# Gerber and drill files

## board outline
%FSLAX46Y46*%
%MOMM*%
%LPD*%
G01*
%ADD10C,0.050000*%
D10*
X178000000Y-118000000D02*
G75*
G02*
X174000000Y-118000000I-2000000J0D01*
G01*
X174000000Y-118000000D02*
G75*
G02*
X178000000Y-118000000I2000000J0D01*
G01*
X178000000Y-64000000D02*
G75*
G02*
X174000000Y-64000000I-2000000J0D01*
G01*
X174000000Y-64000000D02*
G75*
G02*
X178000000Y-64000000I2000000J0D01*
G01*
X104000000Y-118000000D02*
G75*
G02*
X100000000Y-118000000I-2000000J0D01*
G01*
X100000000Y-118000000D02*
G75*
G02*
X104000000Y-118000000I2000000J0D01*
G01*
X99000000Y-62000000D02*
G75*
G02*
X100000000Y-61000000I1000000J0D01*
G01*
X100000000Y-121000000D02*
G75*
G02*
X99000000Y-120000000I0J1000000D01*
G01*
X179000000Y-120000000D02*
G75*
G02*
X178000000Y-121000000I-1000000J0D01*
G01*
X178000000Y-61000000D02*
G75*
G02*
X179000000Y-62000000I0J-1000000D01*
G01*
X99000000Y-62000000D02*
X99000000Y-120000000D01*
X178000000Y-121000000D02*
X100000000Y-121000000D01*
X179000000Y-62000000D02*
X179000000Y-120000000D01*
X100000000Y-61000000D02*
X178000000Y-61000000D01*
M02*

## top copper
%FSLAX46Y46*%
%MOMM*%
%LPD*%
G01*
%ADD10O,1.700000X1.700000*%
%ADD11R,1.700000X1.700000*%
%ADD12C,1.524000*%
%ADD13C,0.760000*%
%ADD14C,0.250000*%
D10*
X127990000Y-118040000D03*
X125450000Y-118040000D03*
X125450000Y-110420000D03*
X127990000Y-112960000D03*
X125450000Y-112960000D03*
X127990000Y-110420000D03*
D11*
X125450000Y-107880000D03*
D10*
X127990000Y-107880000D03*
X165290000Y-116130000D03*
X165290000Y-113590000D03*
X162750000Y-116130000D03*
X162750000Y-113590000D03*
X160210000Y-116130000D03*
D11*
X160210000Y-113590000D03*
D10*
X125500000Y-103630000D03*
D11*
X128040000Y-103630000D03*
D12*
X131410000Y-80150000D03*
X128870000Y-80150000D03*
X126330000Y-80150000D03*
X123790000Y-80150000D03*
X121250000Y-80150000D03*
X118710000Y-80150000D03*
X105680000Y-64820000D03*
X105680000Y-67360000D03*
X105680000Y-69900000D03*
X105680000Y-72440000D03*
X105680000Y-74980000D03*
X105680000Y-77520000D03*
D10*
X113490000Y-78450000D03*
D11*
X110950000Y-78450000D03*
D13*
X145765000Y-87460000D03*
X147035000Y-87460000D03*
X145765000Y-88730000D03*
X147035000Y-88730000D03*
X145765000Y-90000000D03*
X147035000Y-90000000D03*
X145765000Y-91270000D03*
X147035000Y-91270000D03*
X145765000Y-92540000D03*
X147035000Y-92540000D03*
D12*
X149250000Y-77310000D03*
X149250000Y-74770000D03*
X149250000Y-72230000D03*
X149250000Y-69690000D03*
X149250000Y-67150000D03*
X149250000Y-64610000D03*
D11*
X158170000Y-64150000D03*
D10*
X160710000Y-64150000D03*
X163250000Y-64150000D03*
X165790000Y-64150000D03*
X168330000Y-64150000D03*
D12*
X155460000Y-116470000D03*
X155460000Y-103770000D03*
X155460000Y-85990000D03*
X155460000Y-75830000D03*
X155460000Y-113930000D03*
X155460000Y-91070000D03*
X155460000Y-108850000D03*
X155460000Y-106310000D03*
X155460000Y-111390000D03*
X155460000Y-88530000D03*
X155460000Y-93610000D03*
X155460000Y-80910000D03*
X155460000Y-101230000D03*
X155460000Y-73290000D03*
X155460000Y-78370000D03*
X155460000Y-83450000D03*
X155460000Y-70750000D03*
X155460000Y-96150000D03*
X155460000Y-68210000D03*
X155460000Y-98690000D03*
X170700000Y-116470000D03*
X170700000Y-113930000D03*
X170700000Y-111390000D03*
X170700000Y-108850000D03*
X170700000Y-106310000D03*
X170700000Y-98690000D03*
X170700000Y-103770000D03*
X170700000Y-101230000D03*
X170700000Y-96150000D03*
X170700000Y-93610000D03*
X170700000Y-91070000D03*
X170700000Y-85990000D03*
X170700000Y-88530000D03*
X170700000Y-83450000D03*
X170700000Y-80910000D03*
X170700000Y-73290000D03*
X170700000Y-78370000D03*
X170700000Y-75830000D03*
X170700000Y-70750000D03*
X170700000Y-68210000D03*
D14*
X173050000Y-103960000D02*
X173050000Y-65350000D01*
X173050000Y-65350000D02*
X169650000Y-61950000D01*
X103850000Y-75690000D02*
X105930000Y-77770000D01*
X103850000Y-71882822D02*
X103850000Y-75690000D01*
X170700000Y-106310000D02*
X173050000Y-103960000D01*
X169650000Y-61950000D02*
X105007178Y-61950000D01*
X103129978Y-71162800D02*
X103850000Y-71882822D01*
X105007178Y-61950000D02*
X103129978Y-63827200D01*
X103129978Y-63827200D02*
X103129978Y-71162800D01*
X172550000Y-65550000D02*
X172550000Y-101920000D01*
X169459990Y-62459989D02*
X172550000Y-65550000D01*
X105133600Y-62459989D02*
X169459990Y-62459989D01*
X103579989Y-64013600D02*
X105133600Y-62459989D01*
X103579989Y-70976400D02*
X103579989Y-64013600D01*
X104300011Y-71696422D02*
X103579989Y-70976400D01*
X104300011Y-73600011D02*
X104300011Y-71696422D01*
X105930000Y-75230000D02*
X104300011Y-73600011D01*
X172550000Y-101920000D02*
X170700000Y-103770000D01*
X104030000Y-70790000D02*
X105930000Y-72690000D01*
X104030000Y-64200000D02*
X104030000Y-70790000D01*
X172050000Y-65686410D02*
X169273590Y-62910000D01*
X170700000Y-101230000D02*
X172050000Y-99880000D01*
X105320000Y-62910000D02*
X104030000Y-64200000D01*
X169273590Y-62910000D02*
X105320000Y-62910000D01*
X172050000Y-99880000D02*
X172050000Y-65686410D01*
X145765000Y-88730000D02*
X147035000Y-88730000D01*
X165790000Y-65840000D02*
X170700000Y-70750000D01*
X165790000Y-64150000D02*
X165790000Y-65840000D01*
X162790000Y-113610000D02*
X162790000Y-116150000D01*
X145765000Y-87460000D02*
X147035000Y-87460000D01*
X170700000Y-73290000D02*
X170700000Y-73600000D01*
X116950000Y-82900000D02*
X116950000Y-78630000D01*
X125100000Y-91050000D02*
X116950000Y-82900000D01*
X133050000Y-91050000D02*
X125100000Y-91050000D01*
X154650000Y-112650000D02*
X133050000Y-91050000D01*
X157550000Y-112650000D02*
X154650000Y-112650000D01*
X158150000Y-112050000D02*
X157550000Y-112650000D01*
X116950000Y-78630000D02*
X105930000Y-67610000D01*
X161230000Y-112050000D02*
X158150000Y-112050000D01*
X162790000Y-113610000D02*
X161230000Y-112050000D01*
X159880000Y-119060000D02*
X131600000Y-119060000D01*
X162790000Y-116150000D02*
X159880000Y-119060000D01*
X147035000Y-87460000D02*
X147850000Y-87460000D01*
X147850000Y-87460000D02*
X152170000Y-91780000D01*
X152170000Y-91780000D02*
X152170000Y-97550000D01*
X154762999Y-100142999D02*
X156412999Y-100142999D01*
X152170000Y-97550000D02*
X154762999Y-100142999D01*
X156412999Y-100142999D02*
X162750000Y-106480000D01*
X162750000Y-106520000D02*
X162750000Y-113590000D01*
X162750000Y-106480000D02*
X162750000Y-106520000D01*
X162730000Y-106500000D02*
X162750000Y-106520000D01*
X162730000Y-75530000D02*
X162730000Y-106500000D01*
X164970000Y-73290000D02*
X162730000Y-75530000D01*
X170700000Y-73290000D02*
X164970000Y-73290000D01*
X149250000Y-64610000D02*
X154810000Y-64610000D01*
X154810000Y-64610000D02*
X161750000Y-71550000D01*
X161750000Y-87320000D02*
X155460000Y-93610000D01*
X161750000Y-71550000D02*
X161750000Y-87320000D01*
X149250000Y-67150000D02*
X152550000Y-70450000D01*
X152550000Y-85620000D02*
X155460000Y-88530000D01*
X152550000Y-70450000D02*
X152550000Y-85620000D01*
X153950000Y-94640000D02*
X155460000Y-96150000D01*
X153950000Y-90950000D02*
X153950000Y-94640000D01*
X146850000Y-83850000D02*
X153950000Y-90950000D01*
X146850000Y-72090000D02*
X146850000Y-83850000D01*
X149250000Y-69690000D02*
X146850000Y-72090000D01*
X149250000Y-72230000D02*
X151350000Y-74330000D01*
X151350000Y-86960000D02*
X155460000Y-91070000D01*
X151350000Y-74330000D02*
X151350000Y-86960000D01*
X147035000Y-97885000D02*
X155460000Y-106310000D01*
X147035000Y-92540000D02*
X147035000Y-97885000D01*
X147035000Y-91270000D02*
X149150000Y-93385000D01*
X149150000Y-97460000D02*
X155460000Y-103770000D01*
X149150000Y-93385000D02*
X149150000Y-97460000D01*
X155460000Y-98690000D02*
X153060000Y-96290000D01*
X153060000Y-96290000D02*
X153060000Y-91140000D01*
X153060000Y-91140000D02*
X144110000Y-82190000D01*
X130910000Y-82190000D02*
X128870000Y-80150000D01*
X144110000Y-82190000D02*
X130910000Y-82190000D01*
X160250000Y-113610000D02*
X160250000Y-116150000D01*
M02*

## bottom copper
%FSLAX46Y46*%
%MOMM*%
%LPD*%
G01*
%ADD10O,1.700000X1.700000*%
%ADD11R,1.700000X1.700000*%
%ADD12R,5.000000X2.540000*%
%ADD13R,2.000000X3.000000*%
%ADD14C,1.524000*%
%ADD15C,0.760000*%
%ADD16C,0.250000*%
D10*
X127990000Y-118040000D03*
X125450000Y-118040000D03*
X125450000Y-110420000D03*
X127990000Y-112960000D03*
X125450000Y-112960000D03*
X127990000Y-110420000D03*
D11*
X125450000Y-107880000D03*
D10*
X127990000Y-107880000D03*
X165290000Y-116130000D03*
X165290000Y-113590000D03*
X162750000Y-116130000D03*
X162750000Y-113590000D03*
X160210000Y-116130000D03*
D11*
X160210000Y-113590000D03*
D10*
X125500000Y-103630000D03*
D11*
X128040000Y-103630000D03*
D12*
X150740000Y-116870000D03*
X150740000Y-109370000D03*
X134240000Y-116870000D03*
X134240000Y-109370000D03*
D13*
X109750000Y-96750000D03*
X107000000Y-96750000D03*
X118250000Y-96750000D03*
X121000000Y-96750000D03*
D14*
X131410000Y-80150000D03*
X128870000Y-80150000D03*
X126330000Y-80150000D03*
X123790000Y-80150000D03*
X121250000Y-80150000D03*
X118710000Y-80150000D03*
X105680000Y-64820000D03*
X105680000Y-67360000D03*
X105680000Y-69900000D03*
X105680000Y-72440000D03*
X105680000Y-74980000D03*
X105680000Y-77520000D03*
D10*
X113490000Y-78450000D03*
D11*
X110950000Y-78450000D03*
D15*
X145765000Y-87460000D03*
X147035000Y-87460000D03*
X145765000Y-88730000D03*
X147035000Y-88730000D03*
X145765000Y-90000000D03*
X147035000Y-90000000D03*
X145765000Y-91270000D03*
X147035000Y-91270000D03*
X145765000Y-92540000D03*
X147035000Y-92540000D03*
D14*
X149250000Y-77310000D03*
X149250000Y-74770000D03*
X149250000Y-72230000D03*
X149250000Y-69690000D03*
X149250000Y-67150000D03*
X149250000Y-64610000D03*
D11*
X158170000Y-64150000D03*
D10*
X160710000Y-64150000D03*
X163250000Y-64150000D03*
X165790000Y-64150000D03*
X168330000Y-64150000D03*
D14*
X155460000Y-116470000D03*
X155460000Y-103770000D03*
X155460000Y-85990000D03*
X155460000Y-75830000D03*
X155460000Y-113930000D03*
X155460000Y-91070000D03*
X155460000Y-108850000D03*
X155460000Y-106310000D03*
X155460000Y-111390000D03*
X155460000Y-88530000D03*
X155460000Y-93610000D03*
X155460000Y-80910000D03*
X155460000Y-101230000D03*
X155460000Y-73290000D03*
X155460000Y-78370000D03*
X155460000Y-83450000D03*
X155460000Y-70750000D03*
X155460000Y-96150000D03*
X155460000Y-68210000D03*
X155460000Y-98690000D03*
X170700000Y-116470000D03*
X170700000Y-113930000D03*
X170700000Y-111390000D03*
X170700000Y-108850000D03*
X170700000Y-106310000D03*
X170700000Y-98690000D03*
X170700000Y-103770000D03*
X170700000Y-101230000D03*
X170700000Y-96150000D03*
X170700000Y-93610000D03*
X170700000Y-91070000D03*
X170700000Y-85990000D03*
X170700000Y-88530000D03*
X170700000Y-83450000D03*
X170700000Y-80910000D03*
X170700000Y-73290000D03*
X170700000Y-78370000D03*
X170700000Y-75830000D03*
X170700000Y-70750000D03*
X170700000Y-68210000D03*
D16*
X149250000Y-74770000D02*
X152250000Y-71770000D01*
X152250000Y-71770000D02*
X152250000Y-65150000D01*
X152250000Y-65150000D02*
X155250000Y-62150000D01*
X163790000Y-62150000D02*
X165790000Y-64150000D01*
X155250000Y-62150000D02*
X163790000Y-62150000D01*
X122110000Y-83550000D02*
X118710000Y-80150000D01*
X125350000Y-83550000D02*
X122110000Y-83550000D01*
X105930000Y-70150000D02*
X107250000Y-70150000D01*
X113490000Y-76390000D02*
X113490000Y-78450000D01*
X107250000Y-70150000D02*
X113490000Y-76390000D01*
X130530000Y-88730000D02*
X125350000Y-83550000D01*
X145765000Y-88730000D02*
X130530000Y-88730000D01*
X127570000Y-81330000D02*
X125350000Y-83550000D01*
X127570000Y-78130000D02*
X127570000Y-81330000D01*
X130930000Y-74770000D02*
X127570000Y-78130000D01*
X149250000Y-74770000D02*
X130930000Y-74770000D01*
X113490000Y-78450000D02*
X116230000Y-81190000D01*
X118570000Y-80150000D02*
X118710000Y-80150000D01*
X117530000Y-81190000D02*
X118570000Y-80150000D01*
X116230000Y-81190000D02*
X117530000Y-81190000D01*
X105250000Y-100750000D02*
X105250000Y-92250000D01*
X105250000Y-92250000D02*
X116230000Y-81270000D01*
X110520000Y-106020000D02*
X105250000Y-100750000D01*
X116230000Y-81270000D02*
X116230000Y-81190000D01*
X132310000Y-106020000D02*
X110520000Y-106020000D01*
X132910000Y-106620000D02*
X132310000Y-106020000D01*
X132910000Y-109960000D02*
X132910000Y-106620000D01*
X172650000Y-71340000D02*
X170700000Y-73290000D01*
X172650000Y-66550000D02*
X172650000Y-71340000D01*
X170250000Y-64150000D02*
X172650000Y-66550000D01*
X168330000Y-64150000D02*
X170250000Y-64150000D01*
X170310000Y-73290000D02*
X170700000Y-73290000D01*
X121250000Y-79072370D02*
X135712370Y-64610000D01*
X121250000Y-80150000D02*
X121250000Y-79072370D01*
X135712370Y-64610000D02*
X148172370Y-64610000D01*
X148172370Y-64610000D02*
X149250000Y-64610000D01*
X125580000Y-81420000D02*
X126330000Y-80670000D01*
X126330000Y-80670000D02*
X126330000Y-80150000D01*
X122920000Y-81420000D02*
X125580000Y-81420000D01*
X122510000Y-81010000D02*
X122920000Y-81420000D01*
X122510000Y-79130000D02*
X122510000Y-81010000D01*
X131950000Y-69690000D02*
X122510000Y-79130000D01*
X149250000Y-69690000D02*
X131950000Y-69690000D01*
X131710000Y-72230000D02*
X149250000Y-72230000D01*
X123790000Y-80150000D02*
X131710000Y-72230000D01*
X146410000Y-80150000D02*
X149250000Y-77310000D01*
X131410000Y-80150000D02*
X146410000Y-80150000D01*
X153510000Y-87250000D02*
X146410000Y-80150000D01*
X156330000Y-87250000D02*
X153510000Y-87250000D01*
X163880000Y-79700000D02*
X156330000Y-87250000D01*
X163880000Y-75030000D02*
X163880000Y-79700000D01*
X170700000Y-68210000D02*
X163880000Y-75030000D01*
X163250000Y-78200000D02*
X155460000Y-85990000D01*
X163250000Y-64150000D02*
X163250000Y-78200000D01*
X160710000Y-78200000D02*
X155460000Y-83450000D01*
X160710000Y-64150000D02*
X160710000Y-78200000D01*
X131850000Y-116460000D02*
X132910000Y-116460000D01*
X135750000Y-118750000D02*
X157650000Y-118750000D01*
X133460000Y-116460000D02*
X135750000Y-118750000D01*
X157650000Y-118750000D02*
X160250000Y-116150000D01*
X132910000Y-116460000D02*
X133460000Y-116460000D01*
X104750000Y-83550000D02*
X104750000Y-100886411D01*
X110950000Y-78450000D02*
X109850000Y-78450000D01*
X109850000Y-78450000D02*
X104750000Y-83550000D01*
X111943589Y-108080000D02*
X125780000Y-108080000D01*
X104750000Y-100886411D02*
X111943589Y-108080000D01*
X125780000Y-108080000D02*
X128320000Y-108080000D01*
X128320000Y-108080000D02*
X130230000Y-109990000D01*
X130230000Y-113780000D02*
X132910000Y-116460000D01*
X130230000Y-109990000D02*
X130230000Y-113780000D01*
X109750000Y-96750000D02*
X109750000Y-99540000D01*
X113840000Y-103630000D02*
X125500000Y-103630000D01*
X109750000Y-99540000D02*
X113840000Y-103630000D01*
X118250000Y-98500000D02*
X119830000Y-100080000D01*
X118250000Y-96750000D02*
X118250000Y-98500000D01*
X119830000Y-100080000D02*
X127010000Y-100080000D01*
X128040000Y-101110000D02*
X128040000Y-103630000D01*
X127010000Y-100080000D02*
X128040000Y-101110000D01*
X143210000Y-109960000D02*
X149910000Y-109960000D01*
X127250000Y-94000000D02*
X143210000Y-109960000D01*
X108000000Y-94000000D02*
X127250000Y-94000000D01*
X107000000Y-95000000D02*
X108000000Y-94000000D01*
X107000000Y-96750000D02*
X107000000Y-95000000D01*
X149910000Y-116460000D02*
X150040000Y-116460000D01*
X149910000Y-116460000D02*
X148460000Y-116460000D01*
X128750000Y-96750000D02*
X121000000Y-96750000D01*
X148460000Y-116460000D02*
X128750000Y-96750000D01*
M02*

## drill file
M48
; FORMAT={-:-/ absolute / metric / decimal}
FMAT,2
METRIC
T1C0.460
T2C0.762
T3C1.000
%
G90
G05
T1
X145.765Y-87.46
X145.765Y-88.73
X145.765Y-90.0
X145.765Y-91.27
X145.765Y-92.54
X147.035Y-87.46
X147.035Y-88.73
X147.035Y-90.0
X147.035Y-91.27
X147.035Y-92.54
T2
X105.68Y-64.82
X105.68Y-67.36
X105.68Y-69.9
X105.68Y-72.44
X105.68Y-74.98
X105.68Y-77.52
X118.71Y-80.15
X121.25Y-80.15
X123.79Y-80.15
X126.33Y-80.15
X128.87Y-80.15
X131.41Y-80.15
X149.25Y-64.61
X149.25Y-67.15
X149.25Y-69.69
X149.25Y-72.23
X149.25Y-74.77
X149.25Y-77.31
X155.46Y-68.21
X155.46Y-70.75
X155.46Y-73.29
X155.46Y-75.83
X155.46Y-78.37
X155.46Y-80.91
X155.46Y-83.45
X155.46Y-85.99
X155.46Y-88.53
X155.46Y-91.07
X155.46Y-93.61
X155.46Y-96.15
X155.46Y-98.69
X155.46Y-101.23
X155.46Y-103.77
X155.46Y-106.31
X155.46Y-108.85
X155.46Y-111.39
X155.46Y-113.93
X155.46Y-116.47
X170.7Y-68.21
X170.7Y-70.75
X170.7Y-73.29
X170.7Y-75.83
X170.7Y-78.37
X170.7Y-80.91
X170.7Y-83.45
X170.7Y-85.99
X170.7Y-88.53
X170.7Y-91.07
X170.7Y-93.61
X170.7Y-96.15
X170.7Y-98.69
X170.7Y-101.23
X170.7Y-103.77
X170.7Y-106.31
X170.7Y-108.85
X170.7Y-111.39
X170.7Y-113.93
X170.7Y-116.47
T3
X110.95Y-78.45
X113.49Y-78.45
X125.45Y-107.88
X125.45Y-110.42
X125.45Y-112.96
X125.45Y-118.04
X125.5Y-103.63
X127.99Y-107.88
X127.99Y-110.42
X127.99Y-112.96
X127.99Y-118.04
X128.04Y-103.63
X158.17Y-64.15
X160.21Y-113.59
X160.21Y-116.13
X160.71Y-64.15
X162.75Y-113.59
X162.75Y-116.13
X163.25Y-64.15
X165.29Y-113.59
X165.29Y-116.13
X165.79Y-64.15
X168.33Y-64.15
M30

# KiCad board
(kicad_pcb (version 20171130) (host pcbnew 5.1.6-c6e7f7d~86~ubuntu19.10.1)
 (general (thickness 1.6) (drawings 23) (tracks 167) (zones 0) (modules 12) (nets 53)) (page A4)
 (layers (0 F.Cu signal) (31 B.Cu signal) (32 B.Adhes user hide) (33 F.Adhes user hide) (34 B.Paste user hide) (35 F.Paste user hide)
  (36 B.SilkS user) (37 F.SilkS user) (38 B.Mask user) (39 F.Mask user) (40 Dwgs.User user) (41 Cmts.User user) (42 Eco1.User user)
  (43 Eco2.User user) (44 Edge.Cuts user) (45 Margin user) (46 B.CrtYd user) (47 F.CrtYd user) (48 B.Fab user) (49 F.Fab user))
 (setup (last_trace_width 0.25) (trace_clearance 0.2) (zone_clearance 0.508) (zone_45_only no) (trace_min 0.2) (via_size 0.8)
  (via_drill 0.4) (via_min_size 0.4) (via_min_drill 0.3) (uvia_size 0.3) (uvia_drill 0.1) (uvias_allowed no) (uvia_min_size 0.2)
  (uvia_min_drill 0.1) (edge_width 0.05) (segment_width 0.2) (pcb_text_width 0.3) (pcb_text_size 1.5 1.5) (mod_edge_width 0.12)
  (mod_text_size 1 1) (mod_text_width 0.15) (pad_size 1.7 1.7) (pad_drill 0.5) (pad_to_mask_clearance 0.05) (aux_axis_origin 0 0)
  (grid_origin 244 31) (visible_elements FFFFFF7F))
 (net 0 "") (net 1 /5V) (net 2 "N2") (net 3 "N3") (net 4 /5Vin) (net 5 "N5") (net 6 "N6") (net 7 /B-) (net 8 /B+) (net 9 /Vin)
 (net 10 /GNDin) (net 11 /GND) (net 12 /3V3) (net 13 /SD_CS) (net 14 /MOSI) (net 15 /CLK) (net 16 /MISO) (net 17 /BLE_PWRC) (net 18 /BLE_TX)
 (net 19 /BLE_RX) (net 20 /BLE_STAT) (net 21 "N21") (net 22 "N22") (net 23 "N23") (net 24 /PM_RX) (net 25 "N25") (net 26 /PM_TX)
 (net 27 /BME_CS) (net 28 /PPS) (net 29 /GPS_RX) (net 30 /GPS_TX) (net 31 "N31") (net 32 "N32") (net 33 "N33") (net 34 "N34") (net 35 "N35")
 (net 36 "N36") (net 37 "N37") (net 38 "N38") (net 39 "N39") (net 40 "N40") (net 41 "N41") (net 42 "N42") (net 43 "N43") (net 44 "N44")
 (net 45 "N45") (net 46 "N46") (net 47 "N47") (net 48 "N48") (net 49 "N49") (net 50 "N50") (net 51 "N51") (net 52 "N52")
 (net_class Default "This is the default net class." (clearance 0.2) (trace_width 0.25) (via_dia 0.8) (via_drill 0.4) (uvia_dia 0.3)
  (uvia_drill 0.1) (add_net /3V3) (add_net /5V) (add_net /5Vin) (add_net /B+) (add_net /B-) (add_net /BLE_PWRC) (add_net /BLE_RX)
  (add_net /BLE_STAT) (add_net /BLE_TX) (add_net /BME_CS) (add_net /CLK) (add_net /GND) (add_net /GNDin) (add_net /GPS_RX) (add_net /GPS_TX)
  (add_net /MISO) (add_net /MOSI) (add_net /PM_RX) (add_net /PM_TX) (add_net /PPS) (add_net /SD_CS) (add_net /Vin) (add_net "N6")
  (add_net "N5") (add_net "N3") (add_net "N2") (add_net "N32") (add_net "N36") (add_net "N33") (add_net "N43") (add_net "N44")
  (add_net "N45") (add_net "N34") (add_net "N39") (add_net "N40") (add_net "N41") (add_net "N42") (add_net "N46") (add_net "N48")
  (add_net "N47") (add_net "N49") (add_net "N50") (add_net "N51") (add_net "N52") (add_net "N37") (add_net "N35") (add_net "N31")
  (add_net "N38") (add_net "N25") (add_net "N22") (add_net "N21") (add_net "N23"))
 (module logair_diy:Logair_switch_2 (layer B.Cu) (at 126.72 112.96 180)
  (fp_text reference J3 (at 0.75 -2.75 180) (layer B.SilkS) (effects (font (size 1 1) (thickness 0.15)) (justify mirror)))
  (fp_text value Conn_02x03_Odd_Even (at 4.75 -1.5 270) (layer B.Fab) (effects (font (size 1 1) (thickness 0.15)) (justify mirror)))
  (pad "" thru_hole oval (at -1.27 -5.08 180) (size 1.7 1.7) (drill 1) (layers *.Cu *.Mask))
  (pad "" thru_hole oval (at 1.27 -5.08 180) (size 1.7 1.7) (drill 1) (layers *.Cu *.Mask))
  (pad 3 thru_hole oval (at 1.27 2.54 180) (size 1.7 1.7) (drill 1) (layers *.Cu *.Mask) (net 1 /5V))
  (pad 6 thru_hole oval (at -1.27 0 180) (size 1.7 1.7) (drill 1) (layers *.Cu *.Mask) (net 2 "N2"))
  (pad 5 thru_hole oval (at 1.27 0 180) (size 1.7 1.7) (drill 1) (layers *.Cu *.Mask) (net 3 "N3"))
  (pad 4 thru_hole oval (at -1.27 2.54 180) (size 1.7 1.7) (drill 1) (layers *.Cu *.Mask) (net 1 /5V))
  (pad 1 thru_hole rect (at 1.27 5.08 180) (size 1.7 1.7) (drill 1) (layers *.Cu *.Mask) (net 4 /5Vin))
  (pad 2 thru_hole oval (at -1.27 5.08 180) (size 1.7 1.7) (drill 1) (layers *.Cu *.Mask) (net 4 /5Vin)))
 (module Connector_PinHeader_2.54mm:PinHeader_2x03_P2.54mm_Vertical (layer B.Cu) (at 160.21 113.59 270)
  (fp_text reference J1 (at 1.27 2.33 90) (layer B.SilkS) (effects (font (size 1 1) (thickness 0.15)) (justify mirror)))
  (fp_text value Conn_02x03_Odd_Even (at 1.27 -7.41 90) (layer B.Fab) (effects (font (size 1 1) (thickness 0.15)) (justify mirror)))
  (pad 6 thru_hole oval (at 2.54 -5.08 270) (size 1.7 1.7) (drill 1) (layers *.Cu *.Mask) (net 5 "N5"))
  (pad 5 thru_hole oval (at 0 -5.08 270) (size 1.7 1.7) (drill 1) (layers *.Cu *.Mask) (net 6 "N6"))
  (pad 4 thru_hole oval (at 2.54 -2.54 270) (size 1.7 1.7) (drill 1) (layers *.Cu *.Mask) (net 1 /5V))
  (pad 3 thru_hole oval (at 0 -2.54 270) (size 1.7 1.7) (drill 1) (layers *.Cu *.Mask) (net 1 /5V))
  (pad 2 thru_hole oval (at 2.54 0 270) (size 1.7 1.7) (drill 1) (layers *.Cu *.Mask) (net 4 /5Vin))
  (pad 1 thru_hole rect (at 0 0 270) (size 1.7 1.7) (drill 1) (layers *.Cu *.Mask) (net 4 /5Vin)))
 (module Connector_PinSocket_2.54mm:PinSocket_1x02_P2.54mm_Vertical (layer F.Cu) (at 128.04 103.63 270)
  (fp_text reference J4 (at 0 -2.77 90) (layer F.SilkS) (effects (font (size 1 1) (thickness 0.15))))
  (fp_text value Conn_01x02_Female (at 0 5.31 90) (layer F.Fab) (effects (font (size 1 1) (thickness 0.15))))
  (pad 2 thru_hole oval (at 0 2.54 270) (size 1.7 1.7) (drill 1) (layers *.Cu *.Mask) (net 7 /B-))
  (pad 1 thru_hole rect (at 0 0 270) (size 1.7 1.7) (drill 1) (layers *.Cu *.Mask) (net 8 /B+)))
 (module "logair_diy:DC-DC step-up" (layer B.Cu) (at 150.99 113.12 270)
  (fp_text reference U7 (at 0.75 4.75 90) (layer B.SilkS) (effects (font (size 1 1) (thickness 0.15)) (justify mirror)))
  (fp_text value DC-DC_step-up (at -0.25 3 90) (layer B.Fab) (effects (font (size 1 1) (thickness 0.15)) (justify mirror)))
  (pad 4 connect rect (at 3.75 0.25 270) (size 2.54 5) (layers B.Cu B.Mask) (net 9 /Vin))
  (pad 3 connect rect (at -3.75 0.25 270) (size 2.54 5) (layers B.Cu B.Mask) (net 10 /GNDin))
  (pad 2 connect rect (at 3.75 16.75 270) (size 2.54 5) (layers B.Cu B.Mask) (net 4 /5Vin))
  (pad 1 connect rect (at -3.75 16.75 270) (size 2.54 5) (layers B.Cu B.Mask) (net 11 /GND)))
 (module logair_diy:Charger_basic (layer B.Cu) (at 114.25 108.25 180)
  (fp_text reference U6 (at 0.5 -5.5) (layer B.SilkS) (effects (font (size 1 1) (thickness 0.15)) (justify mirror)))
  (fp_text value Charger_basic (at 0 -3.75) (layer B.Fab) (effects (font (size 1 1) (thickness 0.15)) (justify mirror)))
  (pad 3 connect rect (at 4.5 11.5 180) (size 2 3) (layers B.Cu B.Mask) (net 7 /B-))
  (pad 4 connect rect (at 7.25 11.5 180) (size 2 3) (layers B.Cu B.Mask) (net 10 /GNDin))
  (pad 2 connect rect (at -4 11.5 180) (size 2 3) (layers B.Cu B.Mask) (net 8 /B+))
  (pad 1 connect rect (at -6.75 11.5 180) (size 2 3) (layers B.Cu B.Mask) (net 9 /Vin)))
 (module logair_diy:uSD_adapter (layer F.Cu) (at 134.585 62.37 180)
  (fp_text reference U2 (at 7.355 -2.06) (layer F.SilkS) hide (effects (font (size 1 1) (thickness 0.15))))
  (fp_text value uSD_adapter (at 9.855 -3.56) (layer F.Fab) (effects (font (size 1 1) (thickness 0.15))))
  (pad 6 thru_hole circle (at 3.175 -17.78 180) (size 1.524 1.524) (drill 0.762) (layers *.Cu *.Mask) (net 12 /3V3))
  (pad 5 thru_hole circle (at 5.715 -17.78 180) (size 1.524 1.524) (drill 0.762) (layers *.Cu *.Mask) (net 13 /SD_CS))
  (pad 4 thru_hole circle (at 8.255 -17.78 180) (size 1.524 1.524) (drill 0.762) (layers *.Cu *.Mask) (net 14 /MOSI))
  (pad 3 thru_hole circle (at 10.795 -17.78 180) (size 1.524 1.524) (drill 0.762) (layers *.Cu *.Mask) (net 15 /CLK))
  (pad 2 thru_hole circle (at 13.335 -17.78 180) (size 1.524 1.524) (drill 0.762) (layers *.Cu *.Mask) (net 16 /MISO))
  (pad 1 thru_hole circle (at 15.875 -17.78 180) (size 1.524 1.524) (drill 0.762) (layers *.Cu *.Mask) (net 11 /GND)))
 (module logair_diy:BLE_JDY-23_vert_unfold (layer F.Cu) (at 106.95 61.01 270)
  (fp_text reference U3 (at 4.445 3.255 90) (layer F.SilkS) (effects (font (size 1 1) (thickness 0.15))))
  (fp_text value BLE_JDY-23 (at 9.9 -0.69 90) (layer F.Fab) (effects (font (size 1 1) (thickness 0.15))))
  (pad 1 thru_hole circle (at 3.81 1.27 270) (size 1.524 1.524) (drill 0.762) (layers *.Cu *.Mask) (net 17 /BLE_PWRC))
  (pad 2 thru_hole circle (at 6.35 1.27 270) (size 1.524 1.524) (drill 0.762) (layers *.Cu *.Mask) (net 1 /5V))
  (pad 3 thru_hole circle (at 8.89 1.27 270) (size 1.524 1.524) (drill 0.762) (layers *.Cu *.Mask) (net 11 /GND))
  (pad 4 thru_hole circle (at 11.43 1.27 270) (size 1.524 1.524) (drill 0.762) (layers *.Cu *.Mask) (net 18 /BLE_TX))
  (pad 5 thru_hole circle (at 13.97 1.27 270) (size 1.524 1.524) (drill 0.762) (layers *.Cu *.Mask) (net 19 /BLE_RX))
  (pad 6 thru_hole circle (at 16.51 1.27 270) (size 1.524 1.524) (drill 0.762) (layers *.Cu *.Mask) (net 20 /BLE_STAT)))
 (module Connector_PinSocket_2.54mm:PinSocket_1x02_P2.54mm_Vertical (layer F.Cu) (at 110.95 78.45 90)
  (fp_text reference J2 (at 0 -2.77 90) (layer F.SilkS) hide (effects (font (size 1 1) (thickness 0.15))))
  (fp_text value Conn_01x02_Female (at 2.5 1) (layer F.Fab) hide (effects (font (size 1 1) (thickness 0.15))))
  (pad 2 thru_hole oval (at 0 2.54 90) (size 1.7 1.7) (drill 1) (layers *.Cu *.Mask) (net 11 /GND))
  (pad 1 thru_hole rect (at 0 0 90) (size 1.7 1.7) (drill 1) (layers *.Cu *.Mask) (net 4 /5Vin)))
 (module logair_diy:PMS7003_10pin (layer F.Cu) (at 152.25 82.15 270)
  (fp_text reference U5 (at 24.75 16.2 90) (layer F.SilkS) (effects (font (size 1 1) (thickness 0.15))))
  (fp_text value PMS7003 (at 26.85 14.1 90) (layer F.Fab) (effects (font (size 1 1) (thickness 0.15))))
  (pad 2 thru_hole circle (at 5.31 6.485 270) (size 0.76 0.76) (drill 0.46) (layers *.Cu *.Mask) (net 1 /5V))
  (pad 1 thru_hole circle (at 5.31 5.215 270) (size 0.76 0.76) (drill 0.46) (layers *.Cu *.Mask) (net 1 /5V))
  (pad 4 thru_hole circle (at 6.58 6.485 270) (size 0.76 0.76) (drill 0.46) (layers *.Cu *.Mask) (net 11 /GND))
  (pad 3 thru_hole circle (at 6.58 5.215 270) (size 0.76 0.76) (drill 0.46) (layers *.Cu *.Mask) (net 11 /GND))
  (pad 6 thru_hole circle (at 7.85 6.485 270) (size 0.76 0.76) (drill 0.46) (layers *.Cu *.Mask) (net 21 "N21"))
  (pad 5 thru_hole circle (at 7.85 5.215 270) (size 0.76 0.76) (drill 0.46) (layers *.Cu *.Mask) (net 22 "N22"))
  (pad 8 thru_hole circle (at 9.12 6.485 270) (size 0.76 0.76) (drill 0.46) (layers *.Cu *.Mask) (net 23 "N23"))
  (pad 7 thru_hole circle (at 9.12 5.215 270) (size 0.76 0.76) (drill 0.46) (layers *.Cu *.Mask) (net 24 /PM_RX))
  (pad 10 thru_hole circle (at 10.39 6.485 270) (size 0.76 0.76) (drill 0.46) (layers *.Cu *.Mask) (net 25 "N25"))
  (pad 9 thru_hole circle (at 10.39 5.215 270) (size 0.76 0.76) (drill 0.46) (layers *.Cu *.Mask) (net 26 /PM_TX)))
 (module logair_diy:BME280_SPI (layer F.Cu) (at 151.155 62.705 270)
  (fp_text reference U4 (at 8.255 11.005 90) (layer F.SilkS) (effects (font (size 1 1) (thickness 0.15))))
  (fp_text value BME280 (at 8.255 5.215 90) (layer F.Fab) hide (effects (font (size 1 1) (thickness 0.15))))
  (pad 6 thru_hole circle (at 14.605 1.905 270) (size 1.524 1.524) (drill 0.762) (layers *.Cu *.Mask) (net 12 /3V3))
  (pad 5 thru_hole circle (at 12.065 1.905 270) (size 1.524 1.524) (drill 0.762) (layers *.Cu *.Mask) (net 11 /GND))
  (pad 4 thru_hole circle (at 9.525 1.905 270) (size 1.524 1.524) (drill 0.762) (layers *.Cu *.Mask) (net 15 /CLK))
  (pad 3 thru_hole circle (at 6.985 1.905 270) (size 1.524 1.524) (drill 0.762) (layers *.Cu *.Mask) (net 14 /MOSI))
  (pad 2 thru_hole circle (at 4.445 1.905 270) (size 1.524 1.524) (drill 0.762) (layers *.Cu *.Mask) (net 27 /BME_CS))
  (pad 1 thru_hole circle (at 1.905 1.905 270) (size 1.524 1.524) (drill 0.762) (layers *.Cu *.Mask) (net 16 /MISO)))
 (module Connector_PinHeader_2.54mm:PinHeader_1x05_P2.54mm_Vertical (layer F.Cu) (at 158.17 64.15 90)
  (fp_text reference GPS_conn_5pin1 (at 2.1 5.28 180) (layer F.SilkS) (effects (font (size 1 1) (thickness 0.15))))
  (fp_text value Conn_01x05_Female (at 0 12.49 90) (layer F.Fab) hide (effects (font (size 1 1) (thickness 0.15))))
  (pad 1 thru_hole rect (at 0 0 90) (size 1.7 1.7) (drill 1) (layers *.Cu *.Mask) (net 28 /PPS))
  (pad 2 thru_hole oval (at 0 2.54 90) (size 1.7 1.7) (drill 1) (layers *.Cu *.Mask) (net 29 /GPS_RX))
  (pad 3 thru_hole oval (at 0 5.08 90) (size 1.7 1.7) (drill 1) (layers *.Cu *.Mask) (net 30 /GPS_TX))
  (pad 4 thru_hole oval (at 0 7.62 90) (size 1.7 1.7) (drill 1) (layers *.Cu *.Mask) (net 11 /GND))
  (pad 5 thru_hole oval (at 0 10.16 90) (size 1.7 1.7) (drill 1) (layers *.Cu *.Mask) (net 1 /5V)))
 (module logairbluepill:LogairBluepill (layer F.Cu) (at 170.7 68.21 180)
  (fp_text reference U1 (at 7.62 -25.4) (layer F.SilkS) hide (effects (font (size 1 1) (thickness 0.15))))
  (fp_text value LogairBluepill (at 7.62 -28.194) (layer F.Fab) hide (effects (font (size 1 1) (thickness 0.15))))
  (pad GND thru_hole circle (at 15.24 -48.26 270) (size 1.524 1.524) (drill 0.762) (layers *.Cu *.Mask) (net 11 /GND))
  (pad PB10 thru_hole circle (at 15.24 -35.56 270) (size 1.524 1.524) (drill 0.762) (layers *.Cu *.Mask) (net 24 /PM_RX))
  (pad PA3 thru_hole circle (at 15.24 -17.78 270) (size 1.524 1.524) (drill 0.762) (layers *.Cu *.Mask) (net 30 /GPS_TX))
  (pad PC15 thru_hole circle (at 15.24 -7.62 270) (size 1.524 1.524) (drill 0.762) (layers *.Cu *.Mask) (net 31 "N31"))
  (pad GND thru_hole circle (at 15.24 -45.72 270) (size 1.524 1.524) (drill 0.762) (layers *.Cu *.Mask) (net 11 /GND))
  (pad PA5 thru_hole circle (at 15.24 -22.86 270) (size 1.524 1.524) (drill 0.762) (layers *.Cu *.Mask) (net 15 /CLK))
  (pad NRST thru_hole circle (at 15.24 -40.64 270) (size 1.524 1.524) (drill 0.762) (layers *.Cu *.Mask) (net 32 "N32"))
  (pad PB11 thru_hole circle (at 15.24 -38.1 270) (size 1.524 1.524) (drill 0.762) (layers *.Cu *.Mask) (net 26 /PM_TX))
  (pad 3V3 thru_hole circle (at 15.24 -43.18 270) (size 1.524 1.524) (drill 0.762) (layers *.Cu *.Mask) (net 12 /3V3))
  (pad PA4 thru_hole circle (at 15.24 -20.32 270) (size 1.524 1.524) (drill 0.762) (layers *.Cu *.Mask) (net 27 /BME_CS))
  (pad PA6 thru_hole circle (at 15.24 -25.4 270) (size 1.524 1.524) (drill 0.762) (layers *.Cu *.Mask) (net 16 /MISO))
  (pad PA1 thru_hole circle (at 15.24 -12.7 270) (size 1.524 1.524) (drill 0.762) (layers *.Cu *.Mask) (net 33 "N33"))
  (pad PB1 thru_hole circle (at 15.24 -33.02 270) (size 1.524 1.524) (drill 0.762) (layers *.Cu *.Mask) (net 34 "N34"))
  (pad PC14 thru_hole circle (at 15.24 -5.08 270) (size 1.524 1.524) (drill 0.762) (layers *.Cu *.Mask) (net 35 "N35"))
  (pad PA0 thru_hole circle (at 15.24 -10.16 270) (size 1.524 1.524) (drill 0.762) (layers *.Cu *.Mask) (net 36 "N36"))
  (pad PA2 thru_hole circle (at 15.24 -15.24 270) (size 1.524 1.524) (drill 0.762) (layers *.Cu *.Mask) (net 29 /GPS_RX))
  (pad PC13 thru_hole circle (at 15.24 -2.54 270) (size 1.524 1.524) (drill 0.762) (layers *.Cu *.Mask) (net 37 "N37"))
  (pad PA7 thru_hole circle (at 15.24 -27.94 270) (size 1.524 1.524) (drill 0.762) (layers *.Cu *.Mask) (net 14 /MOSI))
  (pad VBAT thru_hole circle (at 15.24 0 270) (size 1.524 1.524) (drill 0.762) (layers *.Cu *.Mask) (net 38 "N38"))
  (pad PB0 thru_hole circle (at 15.24 -30.48 270) (size 1.524 1.524) (drill 0.762) (layers *.Cu *.Mask) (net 13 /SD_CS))
  (pad PB12 thru_hole circle (at 0 -48.26 270) (size 1.524 1.524) (drill 0.762) (layers *.Cu *.Mask) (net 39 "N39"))
  (pad PB13 thru_hole circle (at 0 -45.72 270) (size 1.524 1.524) (drill 0.762) (layers *.Cu *.Mask) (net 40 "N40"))
  (pad PB14 thru_hole circle (at 0 -43.18 270) (size 1.524 1.524) (drill 0.762) (layers *.Cu *.Mask) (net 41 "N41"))
  (pad PB15 thru_hole circle (at 0 -40.64 270) (size 1.524 1.524) (drill 0.762) (layers *.Cu *.Mask) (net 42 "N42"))
  (pad PA8 thru_hole circle (at 0 -38.1 270) (size 1.524 1.524) (drill 0.762) (layers *.Cu *.Mask) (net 20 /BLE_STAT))
  (pad PA11 thru_hole circle (at 0 -30.48 270) (size 1.524 1.524) (drill 0.762) (layers *.Cu *.Mask) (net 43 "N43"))
  (pad PA9 thru_hole circle (at 0 -35.56 270) (size 1.524 1.524) (drill 0.762) (layers *.Cu *.Mask) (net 19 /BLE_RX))
  (pad PA10 thru_hole circle (at 0 -33.02 270) (size 1.524 1.524) (drill 0.762) (layers *.Cu *.Mask) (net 18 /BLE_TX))
  (pad PA12 thru_hole circle (at 0 -27.94 270) (size 1.524 1.524) (drill 0.762) (layers *.Cu *.Mask) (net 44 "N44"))
  (pad PA15 thru_hole circle (at 0 -25.4 270) (size 1.524 1.524) (drill 0.762) (layers *.Cu *.Mask) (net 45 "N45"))
  (pad PB3 thru_hole circle (at 0 -22.86 270) (size 1.524 1.524) (drill 0.762) (layers *.Cu *.Mask) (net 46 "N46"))
  (pad PB5 thru_hole circle (at 0 -17.78 270) (size 1.524 1.524) (drill 0.762) (layers *.Cu *.Mask) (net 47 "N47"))
  (pad PB4 thru_hole circle (at 0 -20.32 270) (size 1.524 1.524) (drill 0.762) (layers *.Cu *.Mask) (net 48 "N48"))
  (pad PB6 thru_hole circle (at 0 -15.24 270) (size 1.524 1.524) (drill 0.762) (layers *.Cu *.Mask) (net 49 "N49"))
  (pad PB7 thru_hole circle (at 0 -12.7 270) (size 1.524 1.524) (drill 0.762) (layers *.Cu *.Mask) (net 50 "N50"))
  (pad 5V thru_hole circle (at 0 -5.08 270) (size 1.524 1.524) (drill 0.762) (layers *.Cu *.Mask) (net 1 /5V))
  (pad PB8 thru_hole circle (at 0 -10.16 270) (size 1.524 1.524) (drill 0.762) (layers *.Cu *.Mask) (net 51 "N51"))
  (pad PB9 thru_hole circle (at 0 -7.62 270) (size 1.524 1.524) (drill 0.762) (layers *.Cu *.Mask) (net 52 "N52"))
  (pad GND thru_hole circle (at 0 -2.54 270) (size 1.524 1.524) (drill 0.762) (layers *.Cu *.Mask) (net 11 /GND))
  (pad 3V3 thru_hole circle (at 0 0 270) (size 1.524 1.524) (drill 0.762) (layers *.Cu *.Mask) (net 12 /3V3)))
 (gr_circle (center 176 118) (end 174 118) (layer Edge.Cuts) (width 0.05))
 (gr_circle (center 176 64) (end 174 64) (layer Edge.Cuts) (width 0.05))
 (gr_circle (center 102 118) (end 100 118) (layer Edge.Cuts) (width 0.05))
 (gr_arc (start 100 62) (end 100 61) (angle -90) (layer Edge.Cuts) (width 0.05))
 (gr_arc (start 100 120) (end 99 120) (angle -90) (layer Edge.Cuts) (width 0.05))
 (gr_arc (start 178 120) (end 178 121) (angle -90) (layer Edge.Cuts) (width 0.05))
 (gr_arc (start 178 62) (end 179 62) (angle -90) (layer Edge.Cuts) (width 0.05))
 (gr_line (start 99 62) (end 99 120) (layer Edge.Cuts) (width 0.05))
 (gr_line (start 178 121) (end 100 121) (layer Edge.Cuts) (width 0.05))
 (gr_line (start 179 62) (end 179 120) (layer Edge.Cuts) (width 0.05))
 (gr_line (start 100 61) (end 178 61) (layer Edge.Cuts) (width 0.05))
 (segment (start 173.05 103.96) (end 173.05 65.35) (width 0.25) (layer F.Cu) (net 20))
 (segment (start 173.05 65.35) (end 169.65 61.95) (width 0.25) (layer F.Cu) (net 20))
 (segment (start 103.85 75.69) (end 105.93 77.77) (width 0.25) (layer F.Cu) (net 20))
 (segment (start 103.85 71.882822) (end 103.85 75.69) (width 0.25) (layer F.Cu) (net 20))
 (segment (start 170.7 106.31) (end 173.05 103.96) (width 0.25) (layer F.Cu) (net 20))
 (segment (start 169.65 61.95) (end 105.007178 61.95) (width 0.25) (layer F.Cu) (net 20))
 (segment (start 103.129978 71.1628) (end 103.85 71.882822) (width 0.25) (layer F.Cu) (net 20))
 (segment (start 105.007178 61.95) (end 103.129978 63.8272) (width 0.25) (layer F.Cu) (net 20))
 (segment (start 103.129978 63.8272) (end 103.129978 71.1628) (width 0.25) (layer F.Cu) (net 20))
 (segment (start 172.55 65.55) (end 172.55 101.92) (width 0.25) (layer F.Cu) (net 19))
 (segment (start 169.45999 62.459989) (end 172.55 65.55) (width 0.25) (layer F.Cu) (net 19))
 (segment (start 105.1336 62.459989) (end 169.45999 62.459989) (width 0.25) (layer F.Cu) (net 19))
 (segment (start 103.579989 64.0136) (end 105.1336 62.459989) (width 0.25) (layer F.Cu) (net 19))
 (segment (start 103.579989 70.9764) (end 103.579989 64.0136) (width 0.25) (layer F.Cu) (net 19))
 (segment (start 104.300011 71.696422) (end 103.579989 70.9764) (width 0.25) (layer F.Cu) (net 19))
 (segment (start 104.300011 73.600011) (end 104.300011 71.696422) (width 0.25) (layer F.Cu) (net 19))
 (segment (start 105.93 75.23) (end 104.300011 73.600011) (width 0.25) (layer F.Cu) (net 19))
 (segment (start 172.55 101.92) (end 170.7 103.77) (width 0.25) (layer F.Cu) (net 19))
 (segment (start 104.03 70.79) (end 105.93 72.69) (width 0.25) (layer F.Cu) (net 18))
 (segment (start 104.03 64.2) (end 104.03 70.79) (width 0.25) (layer F.Cu) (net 18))
 (segment (start 172.05 65.68641) (end 169.27359 62.91) (width 0.25) (layer F.Cu) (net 18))
 (segment (start 170.7 101.23) (end 172.05 99.88) (width 0.25) (layer F.Cu) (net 18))
 (segment (start 105.32 62.91) (end 104.03 64.2) (width 0.25) (layer F.Cu) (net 18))
 (segment (start 169.27359 62.91) (end 105.32 62.91) (width 0.25) (layer F.Cu) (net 18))
 (segment (start 172.05 99.88) (end 172.05 65.68641) (width 0.25) (layer F.Cu) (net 18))
 (segment (start 149.25 74.77) (end 152.25 71.77) (width 0.25) (layer B.Cu) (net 11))
 (segment (start 152.25 71.77) (end 152.25 65.15) (width 0.25) (layer B.Cu) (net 11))
 (segment (start 152.25 65.15) (end 155.25 62.15) (width 0.25) (layer B.Cu) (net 11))
 (segment (start 163.79 62.15) (end 165.79 64.15) (width 0.25) (layer B.Cu) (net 11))
 (segment (start 155.25 62.15) (end 163.79 62.15) (width 0.25) (layer B.Cu) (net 11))
 (segment (start 145.765 88.73) (end 147.035 88.73) (width 0.25) (layer F.Cu) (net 11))
 (segment (start 122.11 83.55) (end 118.71 80.15) (width 0.25) (layer B.Cu) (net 11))
 (segment (start 125.35 83.55) (end 122.11 83.55) (width 0.25) (layer B.Cu) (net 11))
 (segment (start 165.79 65.84) (end 170.7 70.75) (width 0.25) (layer F.Cu) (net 11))
 (segment (start 165.79 64.15) (end 165.79 65.84) (width 0.25) (layer F.Cu) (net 11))
 (segment (start 105.93 70.15) (end 107.25 70.15) (width 0.25) (layer B.Cu) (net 11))
 (segment (start 113.49 76.39) (end 113.49 78.45) (width 0.25) (layer B.Cu) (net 11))
 (segment (start 107.25 70.15) (end 113.49 76.39) (width 0.25) (layer B.Cu) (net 11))
 (segment (start 130.53 88.73) (end 125.35 83.55) (width 0.25) (layer B.Cu) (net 11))
 (segment (start 145.765 88.73) (end 130.53 88.73) (width 0.25) (layer B.Cu) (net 11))
 (segment (start 127.57 81.33) (end 125.35 83.55) (width 0.25) (layer B.Cu) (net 11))
 (segment (start 127.57 78.13) (end 127.57 81.33) (width 0.25) (layer B.Cu) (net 11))
 (segment (start 130.93 74.77) (end 127.57 78.13) (width 0.25) (layer B.Cu) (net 11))
 (segment (start 149.25 74.77) (end 130.93 74.77) (width 0.25) (layer B.Cu) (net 11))
 (segment (start 113.49 78.45) (end 116.23 81.19) (width 0.25) (layer B.Cu) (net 11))
 (segment (start 118.57 80.15) (end 118.71 80.15) (width 0.25) (layer B.Cu) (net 11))
 (segment (start 117.53 81.19) (end 118.57 80.15) (width 0.25) (layer B.Cu) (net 11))
 (segment (start 116.23 81.19) (end 117.53 81.19) (width 0.25) (layer B.Cu) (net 11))
 (segment (start 105.25 100.75) (end 105.25 92.25) (width 0.25) (layer B.Cu) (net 11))
 (segment (start 105.25 92.25) (end 116.23 81.27) (width 0.25) (layer B.Cu) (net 11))
 (segment (start 110.52 106.02) (end 105.25 100.75) (width 0.25) (layer B.Cu) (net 11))
 (segment (start 116.23 81.27) (end 116.23 81.19) (width 0.25) (layer B.Cu) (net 11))
 (segment (start 132.31 106.02) (end 110.52 106.02) (width 0.25) (layer B.Cu) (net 11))
 (segment (start 132.91 106.62) (end 132.31 106.02) (width 0.25) (layer B.Cu) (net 11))
 (segment (start 132.91 109.96) (end 132.91 106.62) (width 0.25) (layer B.Cu) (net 11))
 (segment (start 162.79 113.61) (end 162.79 116.15) (width 0.25) (layer F.Cu) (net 1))
 (segment (start 145.765 87.46) (end 147.035 87.46) (width 0.25) (layer F.Cu) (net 1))
 (segment (start 170.7 73.29) (end 170.7 73.6) (width 0.25) (layer F.Cu) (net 1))
 (segment (start 172.65 71.34) (end 170.7 73.29) (width 0.25) (layer B.Cu) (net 1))
 (segment (start 172.65 66.55) (end 172.65 71.34) (width 0.25) (layer B.Cu) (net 1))
 (segment (start 170.25 64.15) (end 172.65 66.55) (width 0.25) (layer B.Cu) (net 1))
 (segment (start 168.33 64.15) (end 170.25 64.15) (width 0.25) (layer B.Cu) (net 1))
 (segment (start 116.95 82.9) (end 116.95 78.63) (width 0.25) (layer F.Cu) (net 1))
 (segment (start 125.1 91.05) (end 116.95 82.9) (width 0.25) (layer F.Cu) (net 1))
 (segment (start 133.05 91.05) (end 125.1 91.05) (width 0.25) (layer F.Cu) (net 1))
 (segment (start 154.65 112.65) (end 133.05 91.05) (width 0.25) (layer F.Cu) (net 1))
 (segment (start 157.55 112.65) (end 154.65 112.65) (width 0.25) (layer F.Cu) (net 1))
 (segment (start 158.15 112.05) (end 157.55 112.65) (width 0.25) (layer F.Cu) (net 1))
 (segment (start 116.95 78.63) (end 105.93 67.61) (width 0.25) (layer F.Cu) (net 1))
 (segment (start 161.23 112.05) (end 158.15 112.05) (width 0.25) (layer F.Cu) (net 1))
 (segment (start 162.79 113.61) (end 161.23 112.05) (width 0.25) (layer F.Cu) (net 1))
 (segment (start 159.88 119.06) (end 131.6 119.06) (width 0.25) (layer F.Cu) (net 1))
 (segment (start 162.79 116.15) (end 159.88 119.06) (width 0.25) (layer F.Cu) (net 1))
 (segment (start 170.31 73.29) (end 170.7 73.29) (width 0.25) (layer B.Cu) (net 1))
 (segment (start 147.035 87.46) (end 147.85 87.46) (width 0.25) (layer F.Cu) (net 1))
 (segment (start 147.85 87.46) (end 152.17 91.78) (width 0.25) (layer F.Cu) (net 1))
 (segment (start 152.17 91.78) (end 152.17 97.55) (width 0.25) (layer F.Cu) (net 1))
 (segment (start 154.762999 100.142999) (end 156.412999 100.142999) (width 0.25) (layer F.Cu) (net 1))
 (segment (start 152.17 97.55) (end 154.762999 100.142999) (width 0.25) (layer F.Cu) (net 1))
 (segment (start 156.412999 100.142999) (end 162.75 106.48) (width 0.25) (layer F.Cu) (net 1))
 (segment (start 162.75 106.52) (end 162.75 113.59) (width 0.25) (layer F.Cu) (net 1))
 (segment (start 162.75 106.48) (end 162.75 106.52) (width 0.25) (layer F.Cu) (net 1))
 (segment (start 162.73 106.5) (end 162.75 106.52) (width 0.25) (layer F.Cu) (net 1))
 (segment (start 162.73 75.53) (end 162.73 106.5) (width 0.25) (layer F.Cu) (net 1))
 (segment (start 164.97 73.29) (end 162.73 75.53) (width 0.25) (layer F.Cu) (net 1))
 (segment (start 170.7 73.29) (end 164.97 73.29) (width 0.25) (layer F.Cu) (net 1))
 (segment (start 149.25 64.61) (end 154.81 64.61) (width 0.25) (layer F.Cu) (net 16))
 (segment (start 154.81 64.61) (end 161.75 71.55) (width 0.25) (layer F.Cu) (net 16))
 (segment (start 161.75 87.32) (end 155.46 93.61) (width 0.25) (layer F.Cu) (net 16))
 (segment (start 161.75 71.55) (end 161.75 87.32) (width 0.25) (layer F.Cu) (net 16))
 (segment (start 121.25 79.07237) (end 135.71237 64.61) (width 0.25) (layer B.Cu) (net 16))
 (segment (start 121.25 80.15) (end 121.25 79.07237) (width 0.25) (layer B.Cu) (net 16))
 (segment (start 135.71237 64.61) (end 148.17237 64.61) (width 0.25) (layer B.Cu) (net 16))
 (segment (start 148.17237 64.61) (end 149.25 64.61) (width 0.25) (layer B.Cu) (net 16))
 (segment (start 149.25 67.15) (end 152.55 70.45) (width 0.25) (layer F.Cu) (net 27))
 (segment (start 152.55 85.62) (end 155.46 88.53) (width 0.25) (layer F.Cu) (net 27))
 (segment (start 152.55 70.45) (end 152.55 85.62) (width 0.25) (layer F.Cu) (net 27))
 (segment (start 125.58 81.42) (end 126.33 80.67) (width 0.25) (layer B.Cu) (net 14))
 (segment (start 126.33 80.67) (end 126.33 80.15) (width 0.25) (layer B.Cu) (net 14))
 (segment (start 122.92 81.42) (end 125.58 81.42) (width 0.25) (layer B.Cu) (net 14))
 (segment (start 122.51 81.01) (end 122.92 81.42) (width 0.25) (layer B.Cu) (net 14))
 (segment (start 122.51 79.13) (end 122.51 81.01) (width 0.25) (layer B.Cu) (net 14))
 (segment (start 131.95 69.69) (end 122.51 79.13) (width 0.25) (layer B.Cu) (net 14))
 (segment (start 149.25 69.69) (end 131.95 69.69) (width 0.25) (layer B.Cu) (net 14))
 (segment (start 153.95 94.64) (end 155.46 96.15) (width 0.25) (layer F.Cu) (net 14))
 (segment (start 153.95 90.95) (end 153.95 94.64) (width 0.25) (layer F.Cu) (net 14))
 (segment (start 146.85 83.85) (end 153.95 90.95) (width 0.25) (layer F.Cu) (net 14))
 (segment (start 146.85 72.09) (end 146.85 83.85) (width 0.25) (layer F.Cu) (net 14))
 (segment (start 149.25 69.69) (end 146.85 72.09) (width 0.25) (layer F.Cu) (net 14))
 (segment (start 131.71 72.23) (end 149.25 72.23) (width 0.25) (layer B.Cu) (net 15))
 (segment (start 123.79 80.15) (end 131.71 72.23) (width 0.25) (layer B.Cu) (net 15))
 (segment (start 149.25 72.23) (end 151.35 74.33) (width 0.25) (layer F.Cu) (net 15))
 (segment (start 151.35 86.96) (end 155.46 91.07) (width 0.25) (layer F.Cu) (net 15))
 (segment (start 151.35 74.33) (end 151.35 86.96) (width 0.25) (layer F.Cu) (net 15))
 (segment (start 146.41 80.15) (end 149.25 77.31) (width 0.25) (layer B.Cu) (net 12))
 (segment (start 131.41 80.15) (end 146.41 80.15) (width 0.25) (layer B.Cu) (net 12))
 (segment (start 153.51 87.25) (end 146.41 80.15) (width 0.25) (layer B.Cu) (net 12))
 (segment (start 156.33 87.25) (end 153.51 87.25) (width 0.25) (layer B.Cu) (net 12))
 (segment (start 163.88 79.7) (end 156.33 87.25) (width 0.25) (layer B.Cu) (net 12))
 (segment (start 163.88 75.03) (end 163.88 79.7) (width 0.25) (layer B.Cu) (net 12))
 (segment (start 170.7 68.21) (end 163.88 75.03) (width 0.25) (layer B.Cu) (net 12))
 (segment (start 163.25 78.2) (end 155.46 85.99) (width 0.25) (layer B.Cu) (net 30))
 (segment (start 163.25 64.15) (end 163.25 78.2) (width 0.25) (layer B.Cu) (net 30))
 (segment (start 160.71 78.2) (end 155.46 83.45) (width 0.25) (layer B.Cu) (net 29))
 (segment (start 160.71 64.15) (end 160.71 78.2) (width 0.25) (layer B.Cu) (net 29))
 (segment (start 147.035 97.885) (end 155.46 106.31) (width 0.25) (layer F.Cu) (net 26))
 (segment (start 147.035 92.54) (end 147.035 97.885) (width 0.25) (layer F.Cu) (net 26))
 (segment (start 147.035 91.27) (end 149.15 93.385) (width 0.25) (layer F.Cu) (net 24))
 (segment (start 149.15 97.46) (end 155.46 103.77) (width 0.25) (layer F.Cu) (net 24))
 (segment (start 149.15 93.385) (end 149.15 97.46) (width 0.25) (layer F.Cu) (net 24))
 (segment (start 155.46 98.69) (end 153.06 96.29) (width 0.25) (layer F.Cu) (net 13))
 (segment (start 153.06 96.29) (end 153.06 91.14) (width 0.25) (layer F.Cu) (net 13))
 (segment (start 153.06 91.14) (end 144.11 82.19) (width 0.25) (layer F.Cu) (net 13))
 (segment (start 130.91 82.19) (end 128.87 80.15) (width 0.25) (layer F.Cu) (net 13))
 (segment (start 144.11 82.19) (end 130.91 82.19) (width 0.25) (layer F.Cu) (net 13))
 (segment (start 160.25 113.61) (end 160.25 116.15) (width 0.25) (layer F.Cu) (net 4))
 (segment (start 131.85 116.46) (end 132.91 116.46) (width 0.25) (layer B.Cu) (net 4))
 (segment (start 135.75 118.75) (end 157.65 118.75) (width 0.25) (layer B.Cu) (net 4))
 (segment (start 133.46 116.46) (end 135.75 118.75) (width 0.25) (layer B.Cu) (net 4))
 (segment (start 157.65 118.75) (end 160.25 116.15) (width 0.25) (layer B.Cu) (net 4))
 (segment (start 132.91 116.46) (end 133.46 116.46) (width 0.25) (layer B.Cu) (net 4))
 (segment (start 104.75 83.55) (end 104.75 100.886411) (width 0.25) (layer B.Cu) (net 4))
 (segment (start 110.95 78.45) (end 109.85 78.45) (width 0.25) (layer B.Cu) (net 4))
 (segment (start 109.85 78.45) (end 104.75 83.55) (width 0.25) (layer B.Cu) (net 4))
 (segment (start 111.943589 108.08) (end 125.78 108.08) (width 0.25) (layer B.Cu) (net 4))
 (segment (start 104.75 100.886411) (end 111.943589 108.08) (width 0.25) (layer B.Cu) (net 4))
 (segment (start 125.78 108.08) (end 128.32 108.08) (width 0.25) (layer B.Cu) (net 4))
 (segment (start 128.32 108.08) (end 130.23 109.99) (width 0.25) (layer B.Cu) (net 4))
 (segment (start 130.23 113.78) (end 132.91 116.46) (width 0.25) (layer B.Cu) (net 4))
 (segment (start 130.23 109.99) (end 130.23 113.78) (width 0.25) (layer B.Cu) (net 4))
 (segment (start 109.75 96.75) (end 109.75 99.54) (width 0.25) (layer B.Cu) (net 7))
 (segment (start 113.84 103.63) (end 125.5 103.63) (width 0.25) (layer B.Cu) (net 7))
 (segment (start 109.75 99.54) (end 113.84 103.63) (width 0.25) (layer B.Cu) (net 7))
 (segment (start 118.25 98.5) (end 119.83 100.08) (width 0.25) (layer B.Cu) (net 8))
 (segment (start 118.25 96.75) (end 118.25 98.5) (width 0.25) (layer B.Cu) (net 8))
 (segment (start 119.83 100.08) (end 127.01 100.08) (width 0.25) (layer B.Cu) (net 8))
 (segment (start 128.04 101.11) (end 128.04 103.63) (width 0.25) (layer B.Cu) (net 8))
 (segment (start 127.01 100.08) (end 128.04 101.11) (width 0.25) (layer B.Cu) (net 8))
 (segment (start 143.21 109.96) (end 149.91 109.96) (width 0.25) (layer B.Cu) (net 10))
 (segment (start 127.25 94) (end 143.21 109.96) (width 0.25) (layer B.Cu) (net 10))
 (segment (start 108 94) (end 127.25 94) (width 0.25) (layer B.Cu) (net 10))
 (segment (start 107 95) (end 108 94) (width 0.25) (layer B.Cu) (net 10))
 (segment (start 107 96.75) (end 107 95) (width 0.25) (layer B.Cu) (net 10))
 (segment (start 149.91 116.46) (end 150.04 116.46) (width 0.25) (layer B.Cu) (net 9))
 (segment (start 149.91 116.46) (end 148.46 116.46) (width 0.25) (layer B.Cu) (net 9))
 (segment (start 128.75 96.75) (end 121 96.75) (width 0.25) (layer B.Cu) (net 9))
 (segment (start 148.46 116.46) (end 128.75 96.75) (width 0.25) (layer B.Cu) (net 9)))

